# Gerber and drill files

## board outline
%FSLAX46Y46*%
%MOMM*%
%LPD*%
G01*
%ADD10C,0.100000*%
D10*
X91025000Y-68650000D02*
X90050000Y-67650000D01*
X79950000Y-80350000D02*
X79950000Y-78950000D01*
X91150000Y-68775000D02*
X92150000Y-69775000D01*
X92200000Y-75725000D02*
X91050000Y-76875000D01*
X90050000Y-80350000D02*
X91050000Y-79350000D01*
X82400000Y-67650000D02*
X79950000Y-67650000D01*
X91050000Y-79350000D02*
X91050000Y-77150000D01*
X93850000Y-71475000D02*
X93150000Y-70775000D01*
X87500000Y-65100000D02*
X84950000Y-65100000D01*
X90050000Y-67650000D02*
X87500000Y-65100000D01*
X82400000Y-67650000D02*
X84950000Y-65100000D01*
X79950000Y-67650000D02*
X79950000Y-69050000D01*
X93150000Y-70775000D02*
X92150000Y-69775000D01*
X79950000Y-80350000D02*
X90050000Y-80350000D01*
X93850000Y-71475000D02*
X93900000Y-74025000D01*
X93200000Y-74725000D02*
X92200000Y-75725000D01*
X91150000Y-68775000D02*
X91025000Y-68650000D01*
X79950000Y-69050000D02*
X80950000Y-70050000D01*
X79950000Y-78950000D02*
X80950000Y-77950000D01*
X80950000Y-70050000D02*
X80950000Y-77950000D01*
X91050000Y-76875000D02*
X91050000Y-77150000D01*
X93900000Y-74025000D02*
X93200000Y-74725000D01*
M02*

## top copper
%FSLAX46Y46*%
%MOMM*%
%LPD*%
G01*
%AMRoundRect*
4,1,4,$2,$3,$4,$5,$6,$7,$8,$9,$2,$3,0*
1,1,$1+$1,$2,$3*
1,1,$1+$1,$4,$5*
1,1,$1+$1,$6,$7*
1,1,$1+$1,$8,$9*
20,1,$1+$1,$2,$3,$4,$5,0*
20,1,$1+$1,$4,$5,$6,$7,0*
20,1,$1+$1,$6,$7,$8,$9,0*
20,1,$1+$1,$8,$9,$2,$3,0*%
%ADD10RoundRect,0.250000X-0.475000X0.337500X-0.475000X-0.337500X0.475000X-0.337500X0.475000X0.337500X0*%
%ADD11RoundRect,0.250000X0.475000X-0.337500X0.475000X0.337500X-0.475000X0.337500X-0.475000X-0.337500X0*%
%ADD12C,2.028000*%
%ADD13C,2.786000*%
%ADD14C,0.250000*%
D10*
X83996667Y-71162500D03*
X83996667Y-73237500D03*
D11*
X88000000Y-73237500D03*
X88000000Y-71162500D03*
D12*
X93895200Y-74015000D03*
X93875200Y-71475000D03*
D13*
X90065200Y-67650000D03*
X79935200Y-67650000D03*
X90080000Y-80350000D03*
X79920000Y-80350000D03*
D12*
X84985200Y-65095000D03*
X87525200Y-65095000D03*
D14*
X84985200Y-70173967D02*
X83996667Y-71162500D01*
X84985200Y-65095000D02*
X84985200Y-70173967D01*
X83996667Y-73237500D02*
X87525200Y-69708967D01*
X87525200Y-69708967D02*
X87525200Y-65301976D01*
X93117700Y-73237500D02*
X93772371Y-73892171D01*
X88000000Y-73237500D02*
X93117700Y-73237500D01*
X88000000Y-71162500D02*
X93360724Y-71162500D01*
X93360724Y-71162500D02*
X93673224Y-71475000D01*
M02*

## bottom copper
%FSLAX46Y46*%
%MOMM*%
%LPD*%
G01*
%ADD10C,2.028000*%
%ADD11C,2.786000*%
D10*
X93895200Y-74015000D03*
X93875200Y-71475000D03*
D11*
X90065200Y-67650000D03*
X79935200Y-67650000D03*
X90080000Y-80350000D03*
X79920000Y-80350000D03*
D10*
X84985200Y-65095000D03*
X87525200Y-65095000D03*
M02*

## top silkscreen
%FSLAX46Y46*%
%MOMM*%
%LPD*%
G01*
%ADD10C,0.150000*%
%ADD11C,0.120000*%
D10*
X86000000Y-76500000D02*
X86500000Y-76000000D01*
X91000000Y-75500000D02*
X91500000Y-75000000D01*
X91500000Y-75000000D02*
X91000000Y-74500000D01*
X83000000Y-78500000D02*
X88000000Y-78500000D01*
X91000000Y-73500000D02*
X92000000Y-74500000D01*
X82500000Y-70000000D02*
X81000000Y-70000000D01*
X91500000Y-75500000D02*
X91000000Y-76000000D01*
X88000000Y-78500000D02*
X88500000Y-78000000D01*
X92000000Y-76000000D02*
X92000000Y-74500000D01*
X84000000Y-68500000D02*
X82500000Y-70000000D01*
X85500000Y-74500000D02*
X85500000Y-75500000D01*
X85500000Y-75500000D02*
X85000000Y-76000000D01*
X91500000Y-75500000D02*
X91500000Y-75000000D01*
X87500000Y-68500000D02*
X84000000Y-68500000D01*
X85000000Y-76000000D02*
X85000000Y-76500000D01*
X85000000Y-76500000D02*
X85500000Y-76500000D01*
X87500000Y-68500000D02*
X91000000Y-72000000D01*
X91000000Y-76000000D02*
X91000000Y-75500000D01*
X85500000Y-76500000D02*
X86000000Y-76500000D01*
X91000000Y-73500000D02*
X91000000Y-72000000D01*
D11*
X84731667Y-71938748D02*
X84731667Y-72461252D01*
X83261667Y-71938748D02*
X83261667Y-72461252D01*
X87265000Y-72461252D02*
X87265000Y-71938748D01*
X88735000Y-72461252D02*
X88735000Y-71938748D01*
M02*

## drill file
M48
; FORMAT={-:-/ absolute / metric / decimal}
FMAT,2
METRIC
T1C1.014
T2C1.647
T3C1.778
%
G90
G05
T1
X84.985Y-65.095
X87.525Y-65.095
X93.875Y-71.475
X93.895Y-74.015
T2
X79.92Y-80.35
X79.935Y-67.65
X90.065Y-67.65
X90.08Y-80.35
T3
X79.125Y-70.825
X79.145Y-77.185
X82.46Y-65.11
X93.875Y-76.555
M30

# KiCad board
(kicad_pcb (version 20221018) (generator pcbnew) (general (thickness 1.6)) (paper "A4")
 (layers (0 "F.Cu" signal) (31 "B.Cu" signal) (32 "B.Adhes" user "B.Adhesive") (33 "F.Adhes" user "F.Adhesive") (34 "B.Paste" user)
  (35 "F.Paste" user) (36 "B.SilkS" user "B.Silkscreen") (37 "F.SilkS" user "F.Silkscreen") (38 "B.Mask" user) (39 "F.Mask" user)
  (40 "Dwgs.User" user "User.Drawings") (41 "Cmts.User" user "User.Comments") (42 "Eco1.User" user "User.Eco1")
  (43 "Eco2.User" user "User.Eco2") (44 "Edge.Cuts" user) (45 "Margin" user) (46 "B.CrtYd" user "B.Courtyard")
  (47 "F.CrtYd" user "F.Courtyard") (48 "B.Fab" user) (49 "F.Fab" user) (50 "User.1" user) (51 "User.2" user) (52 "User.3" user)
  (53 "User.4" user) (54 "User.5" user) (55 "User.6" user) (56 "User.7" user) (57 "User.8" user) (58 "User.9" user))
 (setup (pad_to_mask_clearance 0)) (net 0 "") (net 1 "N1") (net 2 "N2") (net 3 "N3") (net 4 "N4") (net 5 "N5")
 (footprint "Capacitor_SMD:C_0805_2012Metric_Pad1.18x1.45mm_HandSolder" (layer "F.Cu") (at 83.996667 72.2 -90)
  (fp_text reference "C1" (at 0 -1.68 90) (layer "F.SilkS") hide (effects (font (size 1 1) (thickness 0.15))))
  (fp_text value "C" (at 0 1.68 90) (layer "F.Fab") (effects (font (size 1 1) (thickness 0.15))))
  (fp_line (start -0.261252 -0.735) (end 0.261252 -0.735) (stroke (width 0.12) (type solid)) (layer "F.SilkS"))
  (fp_line (start -0.261252 0.735) (end 0.261252 0.735) (stroke (width 0.12) (type solid)) (layer "F.SilkS"))
  (pad "1" smd roundrect (at -1.0375 0 270) (size 1.175 1.45) (layers "F.Cu" "F.Paste" "F.Mask") (roundrect_rratio 0.212766) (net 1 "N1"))
  (pad "2" smd roundrect (at 1.0375 0 270) (size 1.175 1.45) (layers "F.Cu" "F.Paste" "F.Mask") (roundrect_rratio 0.212766) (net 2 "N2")))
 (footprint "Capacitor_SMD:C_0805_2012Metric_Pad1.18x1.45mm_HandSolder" (layer "F.Cu") (at 88 72.2 90)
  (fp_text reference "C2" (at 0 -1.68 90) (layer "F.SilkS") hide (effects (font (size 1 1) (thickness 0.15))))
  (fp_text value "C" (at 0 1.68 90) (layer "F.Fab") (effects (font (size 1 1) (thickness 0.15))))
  (fp_line (start -0.261252 -0.735) (end 0.261252 -0.735) (stroke (width 0.12) (type solid)) (layer "F.SilkS"))
  (fp_line (start -0.261252 0.735) (end 0.261252 0.735) (stroke (width 0.12) (type solid)) (layer "F.SilkS"))
  (pad "1" smd roundrect (at -1.0375 0 90) (size 1.175 1.45) (layers "F.Cu" "F.Paste" "F.Mask") (roundrect_rratio 0.212766) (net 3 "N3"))
  (pad "2" smd roundrect (at 1.0375 0 90) (size 1.175 1.45) (layers "F.Cu" "F.Paste" "F.Mask") (roundrect_rratio 0.212766) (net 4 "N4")))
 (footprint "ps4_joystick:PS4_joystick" (layer "B.Cu") (at 85 74 -90)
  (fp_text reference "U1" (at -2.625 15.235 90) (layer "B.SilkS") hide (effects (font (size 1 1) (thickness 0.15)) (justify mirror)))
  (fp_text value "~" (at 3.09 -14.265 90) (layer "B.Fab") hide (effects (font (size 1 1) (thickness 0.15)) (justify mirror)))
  (pad "" np_thru_hole circle (at -8.89 2.54 270) (size 1.778 1.778) (drill 1.778) (layers "F&B.Cu" "*.Mask"))
  (pad "" np_thru_hole circle (at -3.175 5.8748 270) (size 1.778 1.778) (drill 1.778) (layers "F&B.Cu" "*.Mask"))
  (pad "" np_thru_hole circle (at 2.555 -8.8752 270) (size 1.778 1.778) (drill 1.778) (layers "F&B.Cu" "*.Mask"))
  (pad "" np_thru_hole circle (at 3.185 5.8548 270) (size 1.778 1.778) (drill 1.778) (layers "F&B.Cu" "*.Mask"))
  (pad "H2" thru_hole circle (at 0.015 -8.8952 270) (size 2.028 2.028) (drill 1.014) (layers "*.Cu" "*.Mask") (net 3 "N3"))
  (pad "H3" thru_hole circle (at -2.525 -8.8752 270) (size 2.028 2.028) (drill 1.014) (layers "*.Cu" "*.Mask") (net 4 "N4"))
  (pad "S" thru_hole circle (at -6.35 -5.0652 270) (size 2.786 2.786) (drill 1.647) (layers "*.Cu" "*.Mask") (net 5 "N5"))
  (pad "S" thru_hole circle (at -6.35 5.0648 270) (size 2.786 2.786) (drill 1.647) (layers "*.Cu" "*.Mask") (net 5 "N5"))
  (pad "S" thru_hole circle (at 6.35 -5.08 270) (size 2.786 2.786) (drill 1.647) (layers "*.Cu" "*.Mask") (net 5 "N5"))
  (pad "S" thru_hole circle (at 6.35 5.08 270) (size 2.786 2.786) (drill 1.647) (layers "*.Cu" "*.Mask") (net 5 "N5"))
  (pad "V2" thru_hole circle (at -8.905 0.0148 270) (size 2.028 2.028) (drill 1.014) (layers "*.Cu" "*.Mask") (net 1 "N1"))
  (pad "V3" thru_hole circle (at -8.905 -2.5252 270) (size 2.028 2.028) (drill 1.014) (layers "*.Cu" "*.Mask") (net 2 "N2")))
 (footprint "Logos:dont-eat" (layer "B.Cu") (at 89.75 77.5 180)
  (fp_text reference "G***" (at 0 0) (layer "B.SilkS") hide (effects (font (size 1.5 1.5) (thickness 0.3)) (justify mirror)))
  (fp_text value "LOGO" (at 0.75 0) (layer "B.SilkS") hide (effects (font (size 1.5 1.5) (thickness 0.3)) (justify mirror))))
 (gr_line (start 86 76.5) (end 86.5 76) (stroke (width 0.15) (type default)) (layer "F.SilkS"))
 (gr_line (start 91 75.5) (end 91.5 75) (stroke (width 0.15) (type default)) (layer "F.SilkS"))
 (gr_line (start 91.5 75) (end 91 74.5) (stroke (width 0.15) (type default)) (layer "F.SilkS"))
 (gr_line (start 83 78.5) (end 88 78.5) (stroke (width 0.15) (type default)) (layer "F.SilkS"))
 (gr_line (start 91 73.5) (end 92 74.5) (stroke (width 0.15) (type default)) (layer "F.SilkS"))
 (gr_line (start 82.5 70) (end 81 70) (stroke (width 0.15) (type default)) (layer "F.SilkS"))
 (gr_line (start 91.5 75.5) (end 91 76) (stroke (width 0.15) (type default)) (layer "F.SilkS"))
 (gr_line (start 88 78.5) (end 88.5 78) (stroke (width 0.15) (type default)) (layer "F.SilkS"))
 (gr_line (start 92 76) (end 92 74.5) (stroke (width 0.15) (type default)) (layer "F.SilkS"))
 (gr_line (start 84 68.5) (end 82.5 70) (stroke (width 0.15) (type default)) (layer "F.SilkS"))
 (gr_line (start 85.5 74.5) (end 85.5 75.5) (stroke (width 0.15) (type default)) (layer "F.SilkS"))
 (gr_line (start 85.5 75.5) (end 85 76) (stroke (width 0.15) (type default)) (layer "F.SilkS"))
 (gr_line (start 91.5 75.5) (end 91.5 75) (stroke (width 0.15) (type default)) (layer "F.SilkS"))
 (gr_line (start 87.5 68.5) (end 84 68.5) (stroke (width 0.15) (type default)) (layer "F.SilkS"))
 (gr_line (start 85 76) (end 85 76.5) (stroke (width 0.15) (type default)) (layer "F.SilkS"))
 (gr_line (start 85 76.5) (end 85.5 76.5) (stroke (width 0.15) (type default)) (layer "F.SilkS"))
 (gr_line (start 87.5 68.5) (end 91 72) (stroke (width 0.15) (type default)) (layer "F.SilkS"))
 (gr_line (start 91 76) (end 91 75.5) (stroke (width 0.15) (type default)) (layer "F.SilkS"))
 (gr_line (start 85.5 76.5) (end 86 76.5) (stroke (width 0.15) (type default)) (layer "F.SilkS"))
 (gr_line (start 91 73.5) (end 91 72) (stroke (width 0.15) (type default)) (layer "F.SilkS"))
 (gr_line (start 91.025 68.65) (end 90.05 67.65) (stroke (width 0.1) (type default)) (layer "Edge.Cuts"))
 (gr_line (start 79.95 80.35) (end 79.95 78.95) (stroke (width 0.1) (type default)) (layer "Edge.Cuts"))
 (gr_line (start 91.15 68.775) (end 92.15 69.775) (stroke (width 0.1) (type default)) (layer "Edge.Cuts"))
 (gr_line (start 92.2 75.725) (end 91.05 76.875) (stroke (width 0.1) (type default)) (layer "Edge.Cuts"))
 (gr_line (start 90.05 80.35) (end 91.05 79.35) (stroke (width 0.1) (type default)) (layer "Edge.Cuts"))
 (gr_line (start 82.4 67.65) (end 79.95 67.65) (stroke (width 0.1) (type default)) (layer "Edge.Cuts"))
 (gr_line (start 91.05 79.35) (end 91.05 77.15) (stroke (width 0.1) (type default)) (layer "Edge.Cuts"))
 (gr_line (start 93.85 71.475) (end 93.15 70.775) (stroke (width 0.1) (type default)) (layer "Edge.Cuts"))
 (gr_line (start 87.5 65.1) (end 84.95 65.1) (stroke (width 0.1) (type default)) (layer "Edge.Cuts"))
 (gr_line (start 90.05 67.65) (end 87.5 65.1) (stroke (width 0.1) (type default)) (layer "Edge.Cuts"))
 (gr_line (start 82.4 67.65) (end 84.95 65.1) (stroke (width 0.1) (type default)) (layer "Edge.Cuts"))
 (gr_line (start 79.95 67.65) (end 79.95 69.05) (stroke (width 0.1) (type default)) (layer "Edge.Cuts"))
 (gr_line (start 93.15 70.775) (end 92.15 69.775) (stroke (width 0.1) (type default)) (layer "Edge.Cuts"))
 (gr_line (start 79.95 80.35) (end 90.05 80.35) (stroke (width 0.1) (type default)) (layer "Edge.Cuts"))
 (gr_line (start 93.85 71.475) (end 93.9 74.025) (stroke (width 0.1) (type default)) (layer "Edge.Cuts"))
 (gr_line (start 93.2 74.725) (end 92.2 75.725) (stroke (width 0.1) (type default)) (layer "Edge.Cuts"))
 (gr_line (start 91.15 68.775) (end 91.025 68.65) (stroke (width 0.1) (type default)) (layer "Edge.Cuts"))
 (gr_line (start 79.95 69.05) (end 80.95 70.05) (stroke (width 0.1) (type default)) (layer "Edge.Cuts"))
 (gr_line (start 79.95 78.95) (end 80.95 77.95) (stroke (width 0.1) (type default)) (layer "Edge.Cuts"))
 (gr_line (start 80.95 70.05) (end 80.95 77.95) (stroke (width 0.1) (type default)) (layer "Edge.Cuts"))
 (gr_line (start 91.05 76.875) (end 91.05 77.15) (stroke (width 0.1) (type default)) (layer "Edge.Cuts"))
 (gr_line (start 93.9 74.025) (end 93.2 74.725) (stroke (width 0.1) (type default)) (layer "Edge.Cuts"))
 (segment (start 84.9852 70.173967) (end 83.996667 71.1625) (width 0.25) (layer "F.Cu") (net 1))
 (segment (start 84.9852 65.095) (end 84.9852 70.173967) (width 0.25) (layer "F.Cu") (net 1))
 (segment (start 83.996667 73.2375) (end 87.5252 69.708967) (width 0.25) (layer "F.Cu") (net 2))
 (segment (start 87.5252 69.708967) (end 87.5252 65.301976) (width 0.25) (layer "F.Cu") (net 2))
 (segment (start 93.1177 73.2375) (end 93.772371 73.892171) (width 0.25) (layer "F.Cu") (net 3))
 (segment (start 88 73.2375) (end 93.1177 73.2375) (width 0.25) (layer "F.Cu") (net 3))
 (segment (start 88 71.1625) (end 93.360724 71.1625) (width 0.25) (layer "F.Cu") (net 4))
 (segment (start 93.360724 71.1625) (end 93.673224 71.475) (width 0.25) (layer "F.Cu") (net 4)))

